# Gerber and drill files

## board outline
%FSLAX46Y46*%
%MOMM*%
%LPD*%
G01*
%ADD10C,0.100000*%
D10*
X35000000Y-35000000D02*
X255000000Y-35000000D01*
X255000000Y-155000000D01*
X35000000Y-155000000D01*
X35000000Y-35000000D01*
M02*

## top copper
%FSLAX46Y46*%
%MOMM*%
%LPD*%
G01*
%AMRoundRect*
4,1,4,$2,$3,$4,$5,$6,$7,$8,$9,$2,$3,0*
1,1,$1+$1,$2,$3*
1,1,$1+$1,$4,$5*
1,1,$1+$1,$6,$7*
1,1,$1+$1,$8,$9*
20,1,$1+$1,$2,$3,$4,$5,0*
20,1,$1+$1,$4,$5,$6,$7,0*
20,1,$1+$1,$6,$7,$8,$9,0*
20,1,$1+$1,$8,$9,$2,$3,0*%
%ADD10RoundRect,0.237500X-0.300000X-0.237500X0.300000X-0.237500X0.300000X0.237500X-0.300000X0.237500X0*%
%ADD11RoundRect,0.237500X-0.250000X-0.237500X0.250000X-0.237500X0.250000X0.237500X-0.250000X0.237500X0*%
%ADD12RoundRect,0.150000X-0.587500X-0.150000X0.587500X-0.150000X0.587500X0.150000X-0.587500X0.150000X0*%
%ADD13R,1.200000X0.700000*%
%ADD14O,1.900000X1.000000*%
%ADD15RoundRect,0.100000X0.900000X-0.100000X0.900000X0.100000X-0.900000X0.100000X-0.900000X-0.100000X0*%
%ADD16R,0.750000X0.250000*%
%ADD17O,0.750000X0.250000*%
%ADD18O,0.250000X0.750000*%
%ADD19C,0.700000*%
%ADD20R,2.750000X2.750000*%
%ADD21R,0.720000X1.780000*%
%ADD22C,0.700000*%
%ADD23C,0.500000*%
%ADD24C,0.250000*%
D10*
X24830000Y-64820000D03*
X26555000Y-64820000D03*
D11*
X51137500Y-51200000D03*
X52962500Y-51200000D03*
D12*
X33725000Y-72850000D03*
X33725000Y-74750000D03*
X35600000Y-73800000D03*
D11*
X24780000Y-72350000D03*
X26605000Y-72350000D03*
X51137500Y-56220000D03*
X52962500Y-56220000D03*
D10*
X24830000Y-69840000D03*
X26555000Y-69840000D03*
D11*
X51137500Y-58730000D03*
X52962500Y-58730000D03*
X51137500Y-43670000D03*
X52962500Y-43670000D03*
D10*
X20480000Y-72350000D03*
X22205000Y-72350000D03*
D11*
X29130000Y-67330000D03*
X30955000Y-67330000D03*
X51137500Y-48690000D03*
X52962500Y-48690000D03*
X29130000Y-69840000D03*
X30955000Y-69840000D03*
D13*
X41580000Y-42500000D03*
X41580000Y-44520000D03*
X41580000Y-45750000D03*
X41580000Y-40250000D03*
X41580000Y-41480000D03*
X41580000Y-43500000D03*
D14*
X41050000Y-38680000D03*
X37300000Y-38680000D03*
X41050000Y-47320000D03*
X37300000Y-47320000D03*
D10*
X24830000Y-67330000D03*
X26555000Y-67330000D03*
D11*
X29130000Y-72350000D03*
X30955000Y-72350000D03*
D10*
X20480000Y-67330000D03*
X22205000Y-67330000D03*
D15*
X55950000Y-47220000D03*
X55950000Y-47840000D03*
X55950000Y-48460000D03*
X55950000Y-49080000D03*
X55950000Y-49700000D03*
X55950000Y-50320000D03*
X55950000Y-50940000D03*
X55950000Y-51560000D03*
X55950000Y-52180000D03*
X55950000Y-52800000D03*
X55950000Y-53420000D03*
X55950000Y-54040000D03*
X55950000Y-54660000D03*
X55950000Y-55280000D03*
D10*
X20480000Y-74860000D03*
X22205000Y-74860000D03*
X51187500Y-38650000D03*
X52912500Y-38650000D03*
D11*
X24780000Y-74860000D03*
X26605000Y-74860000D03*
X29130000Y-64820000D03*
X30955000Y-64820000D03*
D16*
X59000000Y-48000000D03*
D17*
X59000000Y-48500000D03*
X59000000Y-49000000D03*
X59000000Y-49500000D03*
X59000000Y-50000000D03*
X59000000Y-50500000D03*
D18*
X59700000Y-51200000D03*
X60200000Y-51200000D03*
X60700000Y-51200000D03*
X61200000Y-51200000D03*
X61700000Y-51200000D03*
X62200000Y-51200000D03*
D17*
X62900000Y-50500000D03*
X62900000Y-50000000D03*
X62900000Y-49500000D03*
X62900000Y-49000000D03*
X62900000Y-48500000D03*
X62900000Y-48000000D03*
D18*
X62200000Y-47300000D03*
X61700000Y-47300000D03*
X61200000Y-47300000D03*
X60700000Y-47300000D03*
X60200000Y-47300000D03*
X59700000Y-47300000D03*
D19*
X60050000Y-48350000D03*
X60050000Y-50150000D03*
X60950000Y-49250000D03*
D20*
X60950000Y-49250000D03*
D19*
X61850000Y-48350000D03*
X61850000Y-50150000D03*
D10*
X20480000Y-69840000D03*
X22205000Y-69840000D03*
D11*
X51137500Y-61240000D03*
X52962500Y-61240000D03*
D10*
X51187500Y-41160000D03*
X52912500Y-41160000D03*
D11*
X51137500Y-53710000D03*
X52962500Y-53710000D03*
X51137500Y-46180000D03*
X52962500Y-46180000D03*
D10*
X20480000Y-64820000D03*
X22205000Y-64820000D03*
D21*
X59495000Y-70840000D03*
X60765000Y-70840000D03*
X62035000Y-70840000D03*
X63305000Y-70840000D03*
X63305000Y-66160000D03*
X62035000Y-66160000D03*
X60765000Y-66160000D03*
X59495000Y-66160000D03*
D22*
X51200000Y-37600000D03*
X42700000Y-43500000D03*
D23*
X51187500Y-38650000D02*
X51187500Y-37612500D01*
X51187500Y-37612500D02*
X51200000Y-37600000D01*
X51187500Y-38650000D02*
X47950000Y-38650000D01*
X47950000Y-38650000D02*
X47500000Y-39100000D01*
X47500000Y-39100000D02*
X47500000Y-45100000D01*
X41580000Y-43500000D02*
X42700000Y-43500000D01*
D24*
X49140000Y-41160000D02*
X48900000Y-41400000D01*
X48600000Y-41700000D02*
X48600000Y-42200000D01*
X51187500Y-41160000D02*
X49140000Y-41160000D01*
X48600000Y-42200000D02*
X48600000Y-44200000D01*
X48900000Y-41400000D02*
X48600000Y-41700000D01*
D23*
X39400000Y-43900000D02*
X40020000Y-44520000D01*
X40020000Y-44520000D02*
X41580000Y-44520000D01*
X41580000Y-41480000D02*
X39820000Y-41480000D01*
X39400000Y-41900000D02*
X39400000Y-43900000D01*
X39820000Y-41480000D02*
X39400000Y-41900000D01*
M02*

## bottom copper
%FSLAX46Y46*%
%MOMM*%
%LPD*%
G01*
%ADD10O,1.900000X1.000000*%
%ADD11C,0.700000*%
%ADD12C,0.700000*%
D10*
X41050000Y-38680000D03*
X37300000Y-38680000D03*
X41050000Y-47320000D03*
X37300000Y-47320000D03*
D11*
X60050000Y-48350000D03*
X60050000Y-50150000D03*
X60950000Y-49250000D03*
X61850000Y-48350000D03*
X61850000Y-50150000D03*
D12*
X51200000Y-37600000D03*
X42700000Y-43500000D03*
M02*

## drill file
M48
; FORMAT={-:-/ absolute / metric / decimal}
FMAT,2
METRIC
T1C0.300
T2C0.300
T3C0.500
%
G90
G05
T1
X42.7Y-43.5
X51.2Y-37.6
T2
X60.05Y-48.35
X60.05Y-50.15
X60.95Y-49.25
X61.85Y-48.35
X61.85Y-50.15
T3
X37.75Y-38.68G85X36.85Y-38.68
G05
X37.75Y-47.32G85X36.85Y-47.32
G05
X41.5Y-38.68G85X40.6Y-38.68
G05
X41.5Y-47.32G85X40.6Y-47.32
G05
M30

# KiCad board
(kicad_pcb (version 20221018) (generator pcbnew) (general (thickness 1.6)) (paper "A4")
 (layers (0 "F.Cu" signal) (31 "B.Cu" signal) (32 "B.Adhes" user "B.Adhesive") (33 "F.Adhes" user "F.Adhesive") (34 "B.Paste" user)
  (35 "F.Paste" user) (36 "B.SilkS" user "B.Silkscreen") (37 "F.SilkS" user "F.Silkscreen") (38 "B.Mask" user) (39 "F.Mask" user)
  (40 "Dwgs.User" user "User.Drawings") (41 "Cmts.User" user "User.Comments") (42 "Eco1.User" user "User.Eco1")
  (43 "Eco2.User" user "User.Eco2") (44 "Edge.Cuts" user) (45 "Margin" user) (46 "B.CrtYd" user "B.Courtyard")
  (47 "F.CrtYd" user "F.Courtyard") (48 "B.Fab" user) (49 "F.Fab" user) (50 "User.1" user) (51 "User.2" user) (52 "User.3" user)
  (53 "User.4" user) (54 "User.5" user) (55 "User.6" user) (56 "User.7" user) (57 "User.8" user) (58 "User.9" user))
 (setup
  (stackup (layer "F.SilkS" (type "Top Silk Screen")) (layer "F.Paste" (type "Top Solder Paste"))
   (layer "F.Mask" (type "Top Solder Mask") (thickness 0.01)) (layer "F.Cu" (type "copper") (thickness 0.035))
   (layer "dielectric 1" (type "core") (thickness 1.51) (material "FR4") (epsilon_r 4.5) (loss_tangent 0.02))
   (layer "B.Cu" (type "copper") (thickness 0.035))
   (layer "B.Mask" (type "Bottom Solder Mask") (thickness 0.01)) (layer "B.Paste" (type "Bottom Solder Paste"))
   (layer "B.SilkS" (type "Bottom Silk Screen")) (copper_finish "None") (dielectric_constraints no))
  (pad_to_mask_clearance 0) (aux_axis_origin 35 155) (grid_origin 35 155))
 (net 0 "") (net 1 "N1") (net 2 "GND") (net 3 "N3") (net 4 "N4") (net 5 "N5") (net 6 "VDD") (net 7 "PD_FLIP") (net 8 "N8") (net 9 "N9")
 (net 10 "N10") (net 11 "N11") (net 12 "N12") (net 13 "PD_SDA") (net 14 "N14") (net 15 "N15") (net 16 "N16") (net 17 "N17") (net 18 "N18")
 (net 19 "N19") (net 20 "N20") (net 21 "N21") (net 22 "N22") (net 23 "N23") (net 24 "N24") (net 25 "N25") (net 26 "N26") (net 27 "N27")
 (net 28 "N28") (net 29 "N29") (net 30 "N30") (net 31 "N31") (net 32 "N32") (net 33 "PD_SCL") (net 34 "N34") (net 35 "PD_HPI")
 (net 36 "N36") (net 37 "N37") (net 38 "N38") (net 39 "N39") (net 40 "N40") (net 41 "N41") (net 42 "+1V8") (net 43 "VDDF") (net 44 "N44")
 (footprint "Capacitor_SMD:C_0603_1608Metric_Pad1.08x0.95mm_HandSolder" (layer "F.Cu") (at 25.6925 64.82)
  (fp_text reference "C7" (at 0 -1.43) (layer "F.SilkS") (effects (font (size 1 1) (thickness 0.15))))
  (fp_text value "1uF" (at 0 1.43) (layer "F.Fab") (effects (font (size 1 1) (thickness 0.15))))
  (pad "1" smd roundrect (at -0.8625 0) (size 1.075 0.95) (layers "F.Cu" "F.Paste" "F.Mask") (roundrect_rratio 0.25) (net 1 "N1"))
  (pad "2" smd roundrect (at 0.8625 0) (size 1.075 0.95) (layers "F.Cu" "F.Paste" "F.Mask") (roundrect_rratio 0.25) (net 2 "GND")))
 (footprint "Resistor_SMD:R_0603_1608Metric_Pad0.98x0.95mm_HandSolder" (layer "F.Cu") (at 52.05 51.2)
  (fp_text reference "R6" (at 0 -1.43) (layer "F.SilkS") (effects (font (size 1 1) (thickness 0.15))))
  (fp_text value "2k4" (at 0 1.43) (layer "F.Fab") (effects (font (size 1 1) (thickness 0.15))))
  (pad "1" smd roundrect (at -0.9125 0) (size 0.975 0.95) (layers "F.Cu" "F.Paste" "F.Mask") (roundrect_rratio 0.25) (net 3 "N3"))
  (pad "2" smd roundrect (at 0.9125 0) (size 0.975 0.95) (layers "F.Cu" "F.Paste" "F.Mask") (roundrect_rratio 0.25) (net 2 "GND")))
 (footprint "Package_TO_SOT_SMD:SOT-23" (layer "F.Cu") (at 34.6625 73.8)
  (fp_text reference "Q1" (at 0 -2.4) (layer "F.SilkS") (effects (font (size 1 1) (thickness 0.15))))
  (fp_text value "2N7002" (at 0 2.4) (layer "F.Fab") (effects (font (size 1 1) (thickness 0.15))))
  (pad "1" smd roundrect (at -0.9375 -0.95) (size 1.475 0.6) (layers "F.Cu" "F.Paste" "F.Mask") (roundrect_rratio 0.25) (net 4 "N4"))
  (pad "2" smd roundrect (at -0.9375 0.95) (size 1.475 0.6) (layers "F.Cu" "F.Paste" "F.Mask") (roundrect_rratio 0.25) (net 2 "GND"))
  (pad "3" smd roundrect (at 0.9375 0) (size 1.475 0.6) (layers "F.Cu" "F.Paste" "F.Mask") (roundrect_rratio 0.25) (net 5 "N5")))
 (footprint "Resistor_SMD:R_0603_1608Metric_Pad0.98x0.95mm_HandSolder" (layer "F.Cu") (at 25.6925 72.35)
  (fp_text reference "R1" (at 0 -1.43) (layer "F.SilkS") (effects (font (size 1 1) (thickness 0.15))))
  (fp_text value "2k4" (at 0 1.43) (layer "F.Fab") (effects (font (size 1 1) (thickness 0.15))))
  (pad "1" smd roundrect (at -0.9125 0) (size 0.975 0.95) (layers "F.Cu" "F.Paste" "F.Mask") (roundrect_rratio 0.25) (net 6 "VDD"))
  (pad "2" smd roundrect (at 0.9125 0) (size 0.975 0.95) (layers "F.Cu" "F.Paste" "F.Mask") (roundrect_rratio 0.25) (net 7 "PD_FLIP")))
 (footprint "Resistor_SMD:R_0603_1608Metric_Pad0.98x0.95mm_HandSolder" (layer "F.Cu") (at 52.05 56.22)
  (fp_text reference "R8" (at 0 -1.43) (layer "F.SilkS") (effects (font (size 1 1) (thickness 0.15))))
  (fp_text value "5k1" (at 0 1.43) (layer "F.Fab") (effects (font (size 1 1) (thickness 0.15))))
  (pad "1" smd roundrect (at -0.9125 0) (size 0.975 0.95) (layers "F.Cu" "F.Paste" "F.Mask") (roundrect_rratio 0.25) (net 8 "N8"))
  (pad "2" smd roundrect (at 0.9125 0) (size 0.975 0.95) (layers "F.Cu" "F.Paste" "F.Mask") (roundrect_rratio 0.25) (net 2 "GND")))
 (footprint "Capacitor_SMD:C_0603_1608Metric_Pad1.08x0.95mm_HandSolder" (layer "F.Cu") (at 25.6925 69.84)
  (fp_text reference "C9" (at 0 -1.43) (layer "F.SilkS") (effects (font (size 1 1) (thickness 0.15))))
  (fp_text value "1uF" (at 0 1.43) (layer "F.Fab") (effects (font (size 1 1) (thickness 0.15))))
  (pad "1" smd roundrect (at -0.8625 0) (size 1.075 0.95) (layers "F.Cu" "F.Paste" "F.Mask") (roundrect_rratio 0.25) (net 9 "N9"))
  (pad "2" smd roundrect (at 0.8625 0) (size 1.075 0.95) (layers "F.Cu" "F.Paste" "F.Mask") (roundrect_rratio 0.25) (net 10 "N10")))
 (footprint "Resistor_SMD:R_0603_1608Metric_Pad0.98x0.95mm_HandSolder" (layer "F.Cu") (at 52.05 58.73)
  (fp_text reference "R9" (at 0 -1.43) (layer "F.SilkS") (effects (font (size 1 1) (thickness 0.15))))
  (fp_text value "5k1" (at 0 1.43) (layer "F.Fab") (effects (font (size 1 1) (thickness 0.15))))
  (pad "1" smd roundrect (at -0.9125 0) (size 0.975 0.95) (layers "F.Cu" "F.Paste" "F.Mask") (roundrect_rratio 0.25) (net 6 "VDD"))
  (pad "2" smd roundrect (at 0.9125 0) (size 0.975 0.95) (layers "F.Cu" "F.Paste" "F.Mask") (roundrect_rratio 0.25) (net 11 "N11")))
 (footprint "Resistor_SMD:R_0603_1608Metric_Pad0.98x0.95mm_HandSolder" (layer "F.Cu") (at 52.05 43.67)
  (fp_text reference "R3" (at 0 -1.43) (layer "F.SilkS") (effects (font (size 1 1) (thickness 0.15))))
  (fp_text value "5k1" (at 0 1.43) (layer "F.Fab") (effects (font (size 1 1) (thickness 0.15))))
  (pad "1" smd roundrect (at -0.9125 0) (size 0.975 0.95) (layers "F.Cu" "F.Paste" "F.Mask") (roundrect_rratio 0.25) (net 6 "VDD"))
  (pad "2" smd roundrect (at 0.9125 0) (size 0.975 0.95) (layers "F.Cu" "F.Paste" "F.Mask") (roundrect_rratio 0.25) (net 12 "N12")))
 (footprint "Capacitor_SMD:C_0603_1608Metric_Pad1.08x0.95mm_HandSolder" (layer "F.Cu") (at 21.3425 72.35)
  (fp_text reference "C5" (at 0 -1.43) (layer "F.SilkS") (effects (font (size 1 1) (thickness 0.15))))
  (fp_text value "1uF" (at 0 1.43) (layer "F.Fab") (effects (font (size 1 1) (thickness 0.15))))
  (pad "1" smd roundrect (at -0.8625 0) (size 1.075 0.95) (layers "F.Cu" "F.Paste" "F.Mask") (roundrect_rratio 0.25) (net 1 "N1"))
  (pad "2" smd roundrect (at 0.8625 0) (size 1.075 0.95) (layers "F.Cu" "F.Paste" "F.Mask") (roundrect_rratio 0.25) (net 2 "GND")))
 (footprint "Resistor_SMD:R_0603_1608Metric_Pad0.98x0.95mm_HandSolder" (layer "F.Cu") (at 30.0425 67.33)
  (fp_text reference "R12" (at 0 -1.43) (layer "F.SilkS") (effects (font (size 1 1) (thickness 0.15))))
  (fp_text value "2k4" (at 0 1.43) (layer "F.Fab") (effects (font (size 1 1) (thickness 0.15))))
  (pad "1" smd roundrect (at -0.9125 0) (size 0.975 0.95) (layers "F.Cu" "F.Paste" "F.Mask") (roundrect_rratio 0.25) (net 6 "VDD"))
  (pad "2" smd roundrect (at 0.9125 0) (size 0.975 0.95) (layers "F.Cu" "F.Paste" "F.Mask") (roundrect_rratio 0.25) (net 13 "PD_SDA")))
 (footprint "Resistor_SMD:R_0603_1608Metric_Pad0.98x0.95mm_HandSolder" (layer "F.Cu") (at 52.05 48.69)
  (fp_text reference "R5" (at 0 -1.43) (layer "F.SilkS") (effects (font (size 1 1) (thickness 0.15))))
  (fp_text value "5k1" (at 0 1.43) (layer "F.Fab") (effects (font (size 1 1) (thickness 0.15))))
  (pad "1" smd roundrect (at -0.9125 0) (size 0.975 0.95) (layers "F.Cu" "F.Paste" "F.Mask") (roundrect_rratio 0.25) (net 6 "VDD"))
  (pad "2" smd roundrect (at 0.9125 0) (size 0.975 0.95) (layers "F.Cu" "F.Paste" "F.Mask") (roundrect_rratio 0.25) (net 3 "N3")))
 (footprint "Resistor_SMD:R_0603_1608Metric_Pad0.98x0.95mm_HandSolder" (layer "F.Cu") (at 30.0425 69.84)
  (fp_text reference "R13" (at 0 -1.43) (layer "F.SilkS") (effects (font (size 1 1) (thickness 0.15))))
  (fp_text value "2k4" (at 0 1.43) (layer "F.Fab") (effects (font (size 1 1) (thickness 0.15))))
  (pad "1" smd roundrect (at -0.9125 0) (size 0.975 0.95) (layers "F.Cu" "F.Paste" "F.Mask") (roundrect_rratio 0.25) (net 10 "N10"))
  (pad "2" smd roundrect (at 0.9125 0) (size 0.975 0.95) (layers "F.Cu" "F.Paste" "F.Mask") (roundrect_rratio 0.25) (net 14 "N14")))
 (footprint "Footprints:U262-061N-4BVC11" (layer "F.Cu") (at 41.58 43 -90)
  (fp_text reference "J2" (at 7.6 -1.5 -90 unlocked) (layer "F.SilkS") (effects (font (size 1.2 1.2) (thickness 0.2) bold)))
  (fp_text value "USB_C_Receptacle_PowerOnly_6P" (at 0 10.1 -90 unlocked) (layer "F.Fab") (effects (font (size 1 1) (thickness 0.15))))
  (pad "A5" smd rect (at -0.5 0 270) (size 0.7 1.2) (layers "F.Cu" "F.Paste" "F.Mask") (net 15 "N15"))
  (pad "A9" smd rect (at 1.52 0 270) (size 0.7 1.2) (layers "F.Cu" "F.Paste" "F.Mask") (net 1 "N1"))
  (pad "A12" smd rect (at 2.75 0 270) (size 0.7 1.2) (layers "F.Cu" "F.Paste" "F.Mask") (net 2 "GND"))
  (pad "B5" smd rect (at -2.75 0 270) (size 0.7 1.2) (layers "F.Cu" "F.Paste" "F.Mask") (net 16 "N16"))
  (pad "B9" smd rect (at -1.52 0 270) (size 0.7 1.2) (layers "F.Cu" "F.Paste" "F.Mask") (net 1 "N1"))
  (pad "B12" smd rect (at 0.5 0 270) (size 0.7 1.2) (layers "F.Cu" "F.Paste" "F.Mask") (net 2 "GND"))
  (pad "S1" thru_hole oval (at -4.32 0.53 270) (size 1 1.9) (drill oval 0.5 1.4) (layers "*.Cu" "*.Mask") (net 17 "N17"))
  (pad "S1" thru_hole oval (at -4.32 4.28 270) (size 1 1.9) (drill oval 0.5 1.4) (layers "*.Cu" "*.Mask") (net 17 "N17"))
  (pad "S1" thru_hole oval (at 4.32 0.53 270) (size 1 1.9) (drill oval 0.5 1.4) (layers "*.Cu" "*.Mask") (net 17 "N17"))
  (pad "S1" thru_hole oval (at 4.32 4.28 270) (size 1 1.9) (drill oval 0.5 1.4) (layers "*.Cu" "*.Mask") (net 17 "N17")))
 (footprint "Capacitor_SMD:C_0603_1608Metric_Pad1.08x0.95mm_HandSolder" (layer "F.Cu") (at 25.6925 67.33)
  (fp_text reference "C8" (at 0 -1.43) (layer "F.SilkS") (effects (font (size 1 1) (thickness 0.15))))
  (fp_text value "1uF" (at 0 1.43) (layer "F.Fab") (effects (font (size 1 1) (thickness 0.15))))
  (pad "1" smd roundrect (at -0.8625 0) (size 1.075 0.95) (layers "F.Cu" "F.Paste" "F.Mask") (roundrect_rratio 0.25) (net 1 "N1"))
  (pad "2" smd roundrect (at 0.8625 0) (size 1.075 0.95) (layers "F.Cu" "F.Paste" "F.Mask") (roundrect_rratio 0.25) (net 10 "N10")))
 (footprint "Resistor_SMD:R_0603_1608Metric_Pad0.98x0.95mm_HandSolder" (layer "F.Cu") (at 30.0425 72.35)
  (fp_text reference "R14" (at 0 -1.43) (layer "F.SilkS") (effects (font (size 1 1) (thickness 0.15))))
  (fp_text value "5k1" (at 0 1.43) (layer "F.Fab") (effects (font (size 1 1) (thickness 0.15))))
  (pad "1" smd roundrect (at -0.9125 0) (size 0.975 0.95) (layers "F.Cu" "F.Paste" "F.Mask") (roundrect_rratio 0.25) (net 1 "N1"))
  (pad "2" smd roundrect (at 0.9125 0) (size 0.975 0.95) (layers "F.Cu" "F.Paste" "F.Mask") (roundrect_rratio 0.25) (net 10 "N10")))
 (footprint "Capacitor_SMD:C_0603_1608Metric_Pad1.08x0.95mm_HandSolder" (layer "F.Cu") (at 21.3425 67.33)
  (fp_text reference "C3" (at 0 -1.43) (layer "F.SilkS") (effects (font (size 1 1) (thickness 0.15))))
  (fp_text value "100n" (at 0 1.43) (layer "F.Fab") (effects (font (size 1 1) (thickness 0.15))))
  (pad "1" smd roundrect (at -0.8625 0) (size 1.075 0.95) (layers "F.Cu" "F.Paste" "F.Mask") (roundrect_rratio 0.25) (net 6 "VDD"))
  (pad "2" smd roundrect (at 0.8625 0) (size 1.075 0.95) (layers "F.Cu" "F.Paste" "F.Mask") (roundrect_rratio 0.25) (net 2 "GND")))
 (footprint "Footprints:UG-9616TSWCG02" (layer "F.Cu") (at 55.95 51.25)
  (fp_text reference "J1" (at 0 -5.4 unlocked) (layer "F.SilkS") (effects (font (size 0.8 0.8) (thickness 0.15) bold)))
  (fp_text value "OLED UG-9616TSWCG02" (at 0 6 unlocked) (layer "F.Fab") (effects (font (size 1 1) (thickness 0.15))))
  (pad "1" smd roundrect (at 0 -4.03 90) (size 0.4 2) (layers "F.Cu" "F.Paste" "F.Mask") (roundrect_rratio 0.25) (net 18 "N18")
   (thermal_bridge_angle 45))
  (pad "2" smd roundrect (at 0 -3.41 90) (size 0.4 2) (layers "F.Cu" "F.Paste" "F.Mask") (roundrect_rratio 0.25) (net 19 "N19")
   (thermal_bridge_angle 45))
  (pad "3" smd roundrect (at 0 -2.79 90) (size 0.4 2) (layers "F.Cu" "F.Paste" "F.Mask") (roundrect_rratio 0.25) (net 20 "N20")
   (thermal_bridge_angle 45))
  (pad "4" smd roundrect (at 0 -2.17 90) (size 0.4 2) (layers "F.Cu" "F.Paste" "F.Mask") (roundrect_rratio 0.25) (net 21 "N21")
   (thermal_bridge_angle 45))
  (pad "5" smd roundrect (at 0 -1.55 90) (size 0.4 2) (layers "F.Cu" "F.Paste" "F.Mask") (roundrect_rratio 0.25) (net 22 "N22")
   (thermal_bridge_angle 45))
  (pad "6" smd roundrect (at 0 -0.93 90) (size 0.4 2) (layers "F.Cu" "F.Paste" "F.Mask") (roundrect_rratio 0.25) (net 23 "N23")
   (thermal_bridge_angle 45))
  (pad "7" smd roundrect (at 0 -0.31 90) (size 0.4 2) (layers "F.Cu" "F.Paste" "F.Mask") (roundrect_rratio 0.25) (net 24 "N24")
   (thermal_bridge_angle 45))
  (pad "8" smd roundrect (at 0 0.31 90) (size 0.4 2) (layers "F.Cu" "F.Paste" "F.Mask") (roundrect_rratio 0.25) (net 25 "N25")
   (thermal_bridge_angle 45))
  (pad "9" smd roundrect (at 0 0.93 90) (size 0.4 2) (layers "F.Cu" "F.Paste" "F.Mask") (roundrect_rratio 0.25) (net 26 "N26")
   (thermal_bridge_angle 45))
  (pad "10" smd roundrect (at 0 1.55 90) (size 0.4 2) (layers "F.Cu" "F.Paste" "F.Mask") (roundrect_rratio 0.25) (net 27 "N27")
   (thermal_bridge_angle 45))
  (pad "11" smd roundrect (at 0 2.17 90) (size 0.4 2) (layers "F.Cu" "F.Paste" "F.Mask") (roundrect_rratio 0.25) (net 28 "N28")
   (thermal_bridge_angle 45))
  (pad "12" smd roundrect (at 0 2.79 90) (size 0.4 2) (layers "F.Cu" "F.Paste" "F.Mask") (roundrect_rratio 0.25) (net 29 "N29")
   (thermal_bridge_angle 45))
  (pad "13" smd roundrect (at 0 3.41 90) (size 0.4 2) (layers "F.Cu" "F.Paste" "F.Mask") (roundrect_rratio 0.25) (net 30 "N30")
   (thermal_bridge_angle 45))
  (pad "14" smd roundrect (at 0 4.03 90) (size 0.4 2) (layers "F.Cu" "F.Paste" "F.Mask") (roundrect_rratio 0.25) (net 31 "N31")
   (thermal_bridge_angle 45)))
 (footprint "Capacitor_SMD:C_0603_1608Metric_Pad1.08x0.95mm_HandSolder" (layer "F.Cu") (at 21.3425 74.86)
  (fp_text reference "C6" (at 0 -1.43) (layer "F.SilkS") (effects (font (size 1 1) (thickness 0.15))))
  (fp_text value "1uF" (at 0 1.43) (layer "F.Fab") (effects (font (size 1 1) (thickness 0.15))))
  (pad "1" smd roundrect (at -0.8625 0) (size 1.075 0.95) (layers "F.Cu" "F.Paste" "F.Mask") (roundrect_rratio 0.25) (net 1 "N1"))
  (pad "2" smd roundrect (at 0.8625 0) (size 1.075 0.95) (layers "F.Cu" "F.Paste" "F.Mask") (roundrect_rratio 0.25) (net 2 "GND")))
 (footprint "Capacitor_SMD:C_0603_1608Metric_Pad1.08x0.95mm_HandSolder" (layer "F.Cu") (at 52.05 38.65)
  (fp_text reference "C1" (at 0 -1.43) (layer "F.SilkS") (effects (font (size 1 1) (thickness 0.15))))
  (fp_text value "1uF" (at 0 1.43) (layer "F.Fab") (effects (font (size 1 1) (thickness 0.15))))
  (pad "1" smd roundrect (at -0.8625 0) (size 1.075 0.95) (layers "F.Cu" "F.Paste" "F.Mask") (roundrect_rratio 0.25) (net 6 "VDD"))
  (pad "2" smd roundrect (at 0.8625 0) (size 1.075 0.95) (layers "F.Cu" "F.Paste" "F.Mask") (roundrect_rratio 0.25) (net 2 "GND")))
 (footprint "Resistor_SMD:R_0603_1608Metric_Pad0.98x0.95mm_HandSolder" (layer "F.Cu") (at 25.6925 74.86)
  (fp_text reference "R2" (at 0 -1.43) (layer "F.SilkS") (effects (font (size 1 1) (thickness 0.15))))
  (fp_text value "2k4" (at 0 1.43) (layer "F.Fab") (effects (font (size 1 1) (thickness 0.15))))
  (pad "1" smd roundrect (at -0.9125 0) (size 0.975 0.95) (layers "F.Cu" "F.Paste" "F.Mask") (roundrect_rratio 0.25) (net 6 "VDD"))
  (pad "2" smd roundrect (at 0.9125 0) (size 0.975 0.95) (layers "F.Cu" "F.Paste" "F.Mask") (roundrect_rratio 0.25) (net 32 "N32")))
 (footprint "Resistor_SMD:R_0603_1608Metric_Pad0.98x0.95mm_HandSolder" (layer "F.Cu") (at 30.0425 64.82)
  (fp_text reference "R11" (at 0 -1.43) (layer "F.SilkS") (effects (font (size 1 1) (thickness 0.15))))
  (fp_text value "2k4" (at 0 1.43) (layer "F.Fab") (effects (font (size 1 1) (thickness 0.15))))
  (pad "1" smd roundrect (at -0.9125 0) (size 0.975 0.95) (layers "F.Cu" "F.Paste" "F.Mask") (roundrect_rratio 0.25) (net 6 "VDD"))
  (pad "2" smd roundrect (at 0.9125 0) (size 0.975 0.95) (layers "F.Cu" "F.Paste" "F.Mask") (roundrect_rratio 0.25) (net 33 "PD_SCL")))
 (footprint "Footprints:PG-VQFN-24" (layer "F.Cu") (at 60.95 49.25)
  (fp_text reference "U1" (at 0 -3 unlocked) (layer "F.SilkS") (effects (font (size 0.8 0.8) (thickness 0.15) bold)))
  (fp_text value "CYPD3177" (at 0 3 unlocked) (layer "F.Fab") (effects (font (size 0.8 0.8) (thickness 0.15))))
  (pad "1" smd rect (at -1.95 -1.25 90) (size 0.25 0.75) (layers "F.Cu" "F.Paste" "F.Mask") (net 3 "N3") (thermal_bridge_angle 45))
  (pad "2" smd oval (at -1.95 -0.75 90) (size 0.25 0.75) (layers "F.Cu" "F.Paste" "F.Mask") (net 12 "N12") (thermal_bridge_angle 45))
  (pad "3" smd oval (at -1.95 -0.25 90) (size 0.25 0.75) (layers "F.Cu" "F.Paste" "F.Mask") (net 14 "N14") (thermal_bridge_angle 45))
  (pad "4" smd oval (at -1.95 0.25 90) (size 0.25 0.75) (layers "F.Cu" "F.Paste" "F.Mask") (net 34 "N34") (thermal_bridge_angle 45))
  (pad "5" smd oval (at -1.95 0.75 90) (size 0.25 0.75) (layers "F.Cu" "F.Paste" "F.Mask") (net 8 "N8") (thermal_bridge_angle 45))
  (pad "6" smd oval (at -1.95 1.25 90) (size 0.25 0.75) (layers "F.Cu" "F.Paste" "F.Mask") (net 11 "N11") (thermal_bridge_angle 45))
  (pad "7" smd oval (at -1.25 1.95) (size 0.25 0.75) (layers "F.Cu" "F.Paste" "F.Mask") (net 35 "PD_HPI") (thermal_bridge_angle 45))
  (pad "8" smd oval (at -0.75 1.95) (size 0.25 0.75) (layers "F.Cu" "F.Paste" "F.Mask") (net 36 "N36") (thermal_bridge_angle 45))
  (pad "9" smd oval (at -0.25 1.95) (size 0.25 0.75) (layers "F.Cu" "F.Paste" "F.Mask") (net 4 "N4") (thermal_bridge_angle 45))
  (pad "10" smd oval (at 0.25 1.95) (size 0.25 0.75) (layers "F.Cu" "F.Paste" "F.Mask") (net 7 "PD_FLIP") (thermal_bridge_angle 45))
  (pad "11" smd oval (at 0.75 1.95) (size 0.25 0.75) (layers "F.Cu" "F.Paste" "F.Mask") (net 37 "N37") (thermal_bridge_angle 45))
  (pad "12" smd oval (at 1.25 1.95) (size 0.25 0.75) (layers "F.Cu" "F.Paste" "F.Mask") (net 13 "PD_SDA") (thermal_bridge_angle 45))
  (pad "13" smd oval (at 1.95 1.25 270) (size 0.25 0.75) (layers "F.Cu" "F.Paste" "F.Mask") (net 33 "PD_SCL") (thermal_bridge_angle 45))
  (pad "14" smd oval (at 1.95 0.75 270) (size 0.25 0.75) (layers "F.Cu" "F.Paste" "F.Mask") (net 16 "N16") (thermal_bridge_angle 45))
  (pad "15" smd oval (at 1.95 0.25 270) (size 0.25 0.75) (layers "F.Cu" "F.Paste" "F.Mask") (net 15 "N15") (thermal_bridge_angle 45))
  (pad "16" smd oval (at 1.95 -0.25 270) (size 0.25 0.75) (layers "F.Cu" "F.Paste" "F.Mask") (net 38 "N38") (thermal_bridge_angle 45))
  (pad "17" smd oval (at 1.95 -0.75 270) (size 0.25 0.75) (layers "F.Cu" "F.Paste" "F.Mask") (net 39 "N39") (thermal_bridge_angle 45))
  (pad "18" smd oval (at 1.95 -1.25 270) (size 0.25 0.75) (layers "F.Cu" "F.Paste" "F.Mask") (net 1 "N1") (thermal_bridge_angle 45))
  (pad "19" smd oval (at 1.25 -1.95 180) (size 0.25 0.75) (layers "F.Cu" "F.Paste" "F.Mask") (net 2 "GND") (thermal_bridge_angle 45))
  (pad "20" smd oval (at 0.75 -1.95 180) (size 0.25 0.75) (layers "F.Cu" "F.Paste" "F.Mask") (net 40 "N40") (thermal_bridge_angle 45))
  (pad "21" smd oval (at 0.25 -1.95 180) (size 0.25 0.75) (layers "F.Cu" "F.Paste" "F.Mask") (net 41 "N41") (thermal_bridge_angle 45))
  (pad "22" smd oval (at -0.25 -1.95 180) (size 0.25 0.75) (layers "F.Cu" "F.Paste" "F.Mask") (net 2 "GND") (thermal_bridge_angle 45))
  (pad "23" smd oval (at -0.75 -1.95 180) (size 0.25 0.75) (layers "F.Cu" "F.Paste" "F.Mask") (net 6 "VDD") (thermal_bridge_angle 45))
  (pad "24" smd oval (at -1.25 -1.95 180) (size 0.25 0.75) (layers "F.Cu" "F.Paste" "F.Mask") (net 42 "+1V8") (thermal_bridge_angle 45))
  (pad "25" thru_hole circle (at -0.9 -0.9) (size 0.7 0.7) (drill 0.3) (layers "*.Cu" "*.Mask") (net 2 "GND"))
  (pad "25" thru_hole circle (at -0.9 0.9) (size 0.7 0.7) (drill 0.3) (layers "*.Cu" "*.Mask") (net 2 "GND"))
  (pad "25" thru_hole circle (at 0 0) (size 0.7 0.7) (drill 0.3) (layers "*.Cu" "*.Mask") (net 2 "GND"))
  (pad "25" smd rect (at 0 0 180) (size 2.75 2.75) (layers "F.Cu" "F.Paste" "F.Mask") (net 2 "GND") (thermal_bridge_angle 45))
  (pad "25" thru_hole circle (at 0.9 -0.9) (size 0.7 0.7) (drill 0.3) (layers "*.Cu" "*.Mask") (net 2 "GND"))
  (pad "25" thru_hole circle (at 0.9 0.9) (size 0.7 0.7) (drill 0.3) (layers "*.Cu" "*.Mask") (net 2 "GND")))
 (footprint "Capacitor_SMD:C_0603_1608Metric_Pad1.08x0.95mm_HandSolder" (layer "F.Cu") (at 21.3425 69.84)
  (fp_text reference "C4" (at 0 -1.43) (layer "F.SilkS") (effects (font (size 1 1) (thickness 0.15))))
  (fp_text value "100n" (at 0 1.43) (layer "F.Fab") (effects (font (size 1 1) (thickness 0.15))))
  (pad "1" smd roundrect (at -0.8625 0) (size 1.075 0.95) (layers "F.Cu" "F.Paste" "F.Mask") (roundrect_rratio 0.25) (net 6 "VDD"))
  (pad "2" smd roundrect (at 0.8625 0) (size 1.075 0.95) (layers "F.Cu" "F.Paste" "F.Mask") (roundrect_rratio 0.25) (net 2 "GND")))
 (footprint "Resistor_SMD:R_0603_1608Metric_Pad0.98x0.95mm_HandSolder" (layer "F.Cu") (at 52.05 61.24)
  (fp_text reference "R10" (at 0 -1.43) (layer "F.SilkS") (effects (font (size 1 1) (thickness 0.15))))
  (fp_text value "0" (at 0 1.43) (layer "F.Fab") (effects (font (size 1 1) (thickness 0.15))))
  (pad "1" smd roundrect (at -0.9125 0) (size 0.975 0.95) (layers "F.Cu" "F.Paste" "F.Mask") (roundrect_rratio 0.25) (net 11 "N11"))
  (pad "2" smd roundrect (at 0.9125 0) (size 0.975 0.95) (layers "F.Cu" "F.Paste" "F.Mask") (roundrect_rratio 0.25) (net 2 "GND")))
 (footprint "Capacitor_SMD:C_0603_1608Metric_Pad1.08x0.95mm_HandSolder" (layer "F.Cu") (at 52.05 41.16)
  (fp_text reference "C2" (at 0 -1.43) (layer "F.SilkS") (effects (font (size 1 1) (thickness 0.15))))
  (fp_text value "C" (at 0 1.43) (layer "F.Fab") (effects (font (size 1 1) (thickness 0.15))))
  (pad "1" smd roundrect (at -0.8625 0) (size 1.075 0.95) (layers "F.Cu" "F.Paste" "F.Mask") (roundrect_rratio 0.25) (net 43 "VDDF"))
  (pad "2" smd roundrect (at 0.8625 0) (size 1.075 0.95) (layers "F.Cu" "F.Paste" "F.Mask") (roundrect_rratio 0.25) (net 2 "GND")))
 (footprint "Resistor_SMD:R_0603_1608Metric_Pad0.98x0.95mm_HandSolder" (layer "F.Cu") (at 52.05 53.71)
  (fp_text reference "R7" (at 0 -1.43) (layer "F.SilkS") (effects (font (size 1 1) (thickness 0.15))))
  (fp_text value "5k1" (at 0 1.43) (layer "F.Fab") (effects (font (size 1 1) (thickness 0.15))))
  (pad "1" smd roundrect (at -0.9125 0) (size 0.975 0.95) (layers "F.Cu" "F.Paste" "F.Mask") (roundrect_rratio 0.25) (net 6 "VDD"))
  (pad "2" smd roundrect (at 0.9125 0) (size 0.975 0.95) (layers "F.Cu" "F.Paste" "F.Mask") (roundrect_rratio 0.25) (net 8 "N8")))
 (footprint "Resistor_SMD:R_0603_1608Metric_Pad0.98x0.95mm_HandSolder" (layer "F.Cu") (at 52.05 46.18)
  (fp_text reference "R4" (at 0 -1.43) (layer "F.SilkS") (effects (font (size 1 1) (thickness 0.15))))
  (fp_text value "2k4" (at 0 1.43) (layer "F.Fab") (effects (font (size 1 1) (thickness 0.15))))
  (pad "1" smd roundrect (at -0.9125 0) (size 0.975 0.95) (layers "F.Cu" "F.Paste" "F.Mask") (roundrect_rratio 0.25) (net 12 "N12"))
  (pad "2" smd roundrect (at 0.9125 0) (size 0.975 0.95) (layers "F.Cu" "F.Paste" "F.Mask") (roundrect_rratio 0.25) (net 2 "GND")))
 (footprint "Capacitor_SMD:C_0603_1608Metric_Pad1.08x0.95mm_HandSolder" (layer "F.Cu") (at 21.3425 64.82)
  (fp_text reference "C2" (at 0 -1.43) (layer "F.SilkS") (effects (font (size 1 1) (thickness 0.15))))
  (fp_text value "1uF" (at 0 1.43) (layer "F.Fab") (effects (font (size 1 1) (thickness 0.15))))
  (pad "1" smd roundrect (at -0.8625 0) (size 1.075 0.95) (layers "F.Cu" "F.Paste" "F.Mask") (roundrect_rratio 0.25) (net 42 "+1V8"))
  (pad "2" smd roundrect (at 0.8625 0) (size 1.075 0.95) (layers "F.Cu" "F.Paste" "F.Mask") (roundrect_rratio 0.25) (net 2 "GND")))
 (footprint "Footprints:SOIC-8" (layer "F.Cu") (at 61.4 68.5)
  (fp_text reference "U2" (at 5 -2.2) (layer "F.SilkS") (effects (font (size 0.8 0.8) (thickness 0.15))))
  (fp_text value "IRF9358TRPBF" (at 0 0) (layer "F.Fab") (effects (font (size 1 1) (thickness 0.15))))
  (pad "1" smd rect (at -1.905 2.34) (size 0.72 1.78) (layers "F.Cu" "F.Paste" "F.Mask") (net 9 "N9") (thermal_bridge_angle 45))
  (pad "2" smd rect (at -0.635 2.34) (size 0.72 1.78) (layers "F.Cu" "F.Paste" "F.Mask") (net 10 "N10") (thermal_bridge_angle 45))
  (pad "3" smd rect (at 0.635 2.34) (size 0.72 1.78) (layers "F.Cu" "F.Paste" "F.Mask") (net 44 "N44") (thermal_bridge_angle 45))
  (pad "4" smd rect (at 1.905 2.34) (size 0.72 1.78) (layers "F.Cu" "F.Paste" "F.Mask") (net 10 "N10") (thermal_bridge_angle 45))
  (pad "5" smd rect (at 1.905 -2.34) (size 0.72 1.78) (layers "F.Cu" "F.Paste" "F.Mask") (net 1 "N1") (thermal_bridge_angle 45))
  (pad "6" smd rect (at 0.635 -2.34) (size 0.72 1.78) (layers "F.Cu" "F.Paste" "F.Mask") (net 1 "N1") (thermal_bridge_angle 45))
  (pad "7" smd rect (at -0.635 -2.34) (size 0.72 1.78) (layers "F.Cu" "F.Paste" "F.Mask") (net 44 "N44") (thermal_bridge_angle 45))
  (pad "8" smd rect (at -1.905 -2.34) (size 0.72 1.78) (layers "F.Cu" "F.Paste" "F.Mask") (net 44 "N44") (thermal_bridge_angle 45)))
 (gr_rect (start 35 35) (end 255 155) (stroke (width 0.1) (type default)) (fill none) (layer "Edge.Cuts"))
 (segment (start 51.1875 38.65) (end 51.1875 37.6125) (width 0.5) (layer "F.Cu") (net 6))
 (segment (start 51.1875 37.6125) (end 51.2 37.6) (width 0.5) (layer "F.Cu") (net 6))
 (segment (start 51.1875 38.65) (end 47.95 38.65) (width 0.5) (layer "F.Cu") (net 6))
 (segment (start 47.95 38.65) (end 47.5 39.1) (width 0.5) (layer "F.Cu") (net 6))
 (segment (start 47.5 39.1) (end 47.5 45.1) (width 0.5) (layer "F.Cu") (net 6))
 (via (at 51.2 37.6) (size 0.7) (drill 0.3) (layers "F.Cu" "B.Cu") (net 6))
 (segment (start 41.58 43.5) (end 42.7 43.5) (width 0.5) (layer "F.Cu") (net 2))
 (via (at 42.7 43.5) (size 0.7) (drill 0.3) (layers "F.Cu" "B.Cu") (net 2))
 (segment (start 49.14 41.16) (end 48.9 41.4) (width 0.25) (layer "F.Cu") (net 43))
 (segment (start 48.6 41.7) (end 48.6 42.2) (width 0.25) (layer "F.Cu") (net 43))
 (segment (start 51.1875 41.16) (end 49.14 41.16) (width 0.25) (layer "F.Cu") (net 43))
 (segment (start 48.6 42.2) (end 48.6 44.2) (width 0.25) (layer "F.Cu") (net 43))
 (segment (start 48.9 41.4) (end 48.6 41.7) (width 0.25) (layer "F.Cu") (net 43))
 (segment (start 39.4 43.9) (end 40.02 44.52) (width 0.5) (layer "F.Cu") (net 1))
 (segment (start 40.02 44.52) (end 41.58 44.52) (width 0.5) (layer "F.Cu") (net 1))
 (segment (start 41.58 41.48) (end 39.82 41.48) (width 0.5) (layer "F.Cu") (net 1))
 (segment (start 39.4 41.9) (end 39.4 43.9) (width 0.5) (layer "F.Cu") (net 1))
 (segment (start 39.82 41.48) (end 39.4 41.9) (width 0.5) (layer "F.Cu") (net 1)))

